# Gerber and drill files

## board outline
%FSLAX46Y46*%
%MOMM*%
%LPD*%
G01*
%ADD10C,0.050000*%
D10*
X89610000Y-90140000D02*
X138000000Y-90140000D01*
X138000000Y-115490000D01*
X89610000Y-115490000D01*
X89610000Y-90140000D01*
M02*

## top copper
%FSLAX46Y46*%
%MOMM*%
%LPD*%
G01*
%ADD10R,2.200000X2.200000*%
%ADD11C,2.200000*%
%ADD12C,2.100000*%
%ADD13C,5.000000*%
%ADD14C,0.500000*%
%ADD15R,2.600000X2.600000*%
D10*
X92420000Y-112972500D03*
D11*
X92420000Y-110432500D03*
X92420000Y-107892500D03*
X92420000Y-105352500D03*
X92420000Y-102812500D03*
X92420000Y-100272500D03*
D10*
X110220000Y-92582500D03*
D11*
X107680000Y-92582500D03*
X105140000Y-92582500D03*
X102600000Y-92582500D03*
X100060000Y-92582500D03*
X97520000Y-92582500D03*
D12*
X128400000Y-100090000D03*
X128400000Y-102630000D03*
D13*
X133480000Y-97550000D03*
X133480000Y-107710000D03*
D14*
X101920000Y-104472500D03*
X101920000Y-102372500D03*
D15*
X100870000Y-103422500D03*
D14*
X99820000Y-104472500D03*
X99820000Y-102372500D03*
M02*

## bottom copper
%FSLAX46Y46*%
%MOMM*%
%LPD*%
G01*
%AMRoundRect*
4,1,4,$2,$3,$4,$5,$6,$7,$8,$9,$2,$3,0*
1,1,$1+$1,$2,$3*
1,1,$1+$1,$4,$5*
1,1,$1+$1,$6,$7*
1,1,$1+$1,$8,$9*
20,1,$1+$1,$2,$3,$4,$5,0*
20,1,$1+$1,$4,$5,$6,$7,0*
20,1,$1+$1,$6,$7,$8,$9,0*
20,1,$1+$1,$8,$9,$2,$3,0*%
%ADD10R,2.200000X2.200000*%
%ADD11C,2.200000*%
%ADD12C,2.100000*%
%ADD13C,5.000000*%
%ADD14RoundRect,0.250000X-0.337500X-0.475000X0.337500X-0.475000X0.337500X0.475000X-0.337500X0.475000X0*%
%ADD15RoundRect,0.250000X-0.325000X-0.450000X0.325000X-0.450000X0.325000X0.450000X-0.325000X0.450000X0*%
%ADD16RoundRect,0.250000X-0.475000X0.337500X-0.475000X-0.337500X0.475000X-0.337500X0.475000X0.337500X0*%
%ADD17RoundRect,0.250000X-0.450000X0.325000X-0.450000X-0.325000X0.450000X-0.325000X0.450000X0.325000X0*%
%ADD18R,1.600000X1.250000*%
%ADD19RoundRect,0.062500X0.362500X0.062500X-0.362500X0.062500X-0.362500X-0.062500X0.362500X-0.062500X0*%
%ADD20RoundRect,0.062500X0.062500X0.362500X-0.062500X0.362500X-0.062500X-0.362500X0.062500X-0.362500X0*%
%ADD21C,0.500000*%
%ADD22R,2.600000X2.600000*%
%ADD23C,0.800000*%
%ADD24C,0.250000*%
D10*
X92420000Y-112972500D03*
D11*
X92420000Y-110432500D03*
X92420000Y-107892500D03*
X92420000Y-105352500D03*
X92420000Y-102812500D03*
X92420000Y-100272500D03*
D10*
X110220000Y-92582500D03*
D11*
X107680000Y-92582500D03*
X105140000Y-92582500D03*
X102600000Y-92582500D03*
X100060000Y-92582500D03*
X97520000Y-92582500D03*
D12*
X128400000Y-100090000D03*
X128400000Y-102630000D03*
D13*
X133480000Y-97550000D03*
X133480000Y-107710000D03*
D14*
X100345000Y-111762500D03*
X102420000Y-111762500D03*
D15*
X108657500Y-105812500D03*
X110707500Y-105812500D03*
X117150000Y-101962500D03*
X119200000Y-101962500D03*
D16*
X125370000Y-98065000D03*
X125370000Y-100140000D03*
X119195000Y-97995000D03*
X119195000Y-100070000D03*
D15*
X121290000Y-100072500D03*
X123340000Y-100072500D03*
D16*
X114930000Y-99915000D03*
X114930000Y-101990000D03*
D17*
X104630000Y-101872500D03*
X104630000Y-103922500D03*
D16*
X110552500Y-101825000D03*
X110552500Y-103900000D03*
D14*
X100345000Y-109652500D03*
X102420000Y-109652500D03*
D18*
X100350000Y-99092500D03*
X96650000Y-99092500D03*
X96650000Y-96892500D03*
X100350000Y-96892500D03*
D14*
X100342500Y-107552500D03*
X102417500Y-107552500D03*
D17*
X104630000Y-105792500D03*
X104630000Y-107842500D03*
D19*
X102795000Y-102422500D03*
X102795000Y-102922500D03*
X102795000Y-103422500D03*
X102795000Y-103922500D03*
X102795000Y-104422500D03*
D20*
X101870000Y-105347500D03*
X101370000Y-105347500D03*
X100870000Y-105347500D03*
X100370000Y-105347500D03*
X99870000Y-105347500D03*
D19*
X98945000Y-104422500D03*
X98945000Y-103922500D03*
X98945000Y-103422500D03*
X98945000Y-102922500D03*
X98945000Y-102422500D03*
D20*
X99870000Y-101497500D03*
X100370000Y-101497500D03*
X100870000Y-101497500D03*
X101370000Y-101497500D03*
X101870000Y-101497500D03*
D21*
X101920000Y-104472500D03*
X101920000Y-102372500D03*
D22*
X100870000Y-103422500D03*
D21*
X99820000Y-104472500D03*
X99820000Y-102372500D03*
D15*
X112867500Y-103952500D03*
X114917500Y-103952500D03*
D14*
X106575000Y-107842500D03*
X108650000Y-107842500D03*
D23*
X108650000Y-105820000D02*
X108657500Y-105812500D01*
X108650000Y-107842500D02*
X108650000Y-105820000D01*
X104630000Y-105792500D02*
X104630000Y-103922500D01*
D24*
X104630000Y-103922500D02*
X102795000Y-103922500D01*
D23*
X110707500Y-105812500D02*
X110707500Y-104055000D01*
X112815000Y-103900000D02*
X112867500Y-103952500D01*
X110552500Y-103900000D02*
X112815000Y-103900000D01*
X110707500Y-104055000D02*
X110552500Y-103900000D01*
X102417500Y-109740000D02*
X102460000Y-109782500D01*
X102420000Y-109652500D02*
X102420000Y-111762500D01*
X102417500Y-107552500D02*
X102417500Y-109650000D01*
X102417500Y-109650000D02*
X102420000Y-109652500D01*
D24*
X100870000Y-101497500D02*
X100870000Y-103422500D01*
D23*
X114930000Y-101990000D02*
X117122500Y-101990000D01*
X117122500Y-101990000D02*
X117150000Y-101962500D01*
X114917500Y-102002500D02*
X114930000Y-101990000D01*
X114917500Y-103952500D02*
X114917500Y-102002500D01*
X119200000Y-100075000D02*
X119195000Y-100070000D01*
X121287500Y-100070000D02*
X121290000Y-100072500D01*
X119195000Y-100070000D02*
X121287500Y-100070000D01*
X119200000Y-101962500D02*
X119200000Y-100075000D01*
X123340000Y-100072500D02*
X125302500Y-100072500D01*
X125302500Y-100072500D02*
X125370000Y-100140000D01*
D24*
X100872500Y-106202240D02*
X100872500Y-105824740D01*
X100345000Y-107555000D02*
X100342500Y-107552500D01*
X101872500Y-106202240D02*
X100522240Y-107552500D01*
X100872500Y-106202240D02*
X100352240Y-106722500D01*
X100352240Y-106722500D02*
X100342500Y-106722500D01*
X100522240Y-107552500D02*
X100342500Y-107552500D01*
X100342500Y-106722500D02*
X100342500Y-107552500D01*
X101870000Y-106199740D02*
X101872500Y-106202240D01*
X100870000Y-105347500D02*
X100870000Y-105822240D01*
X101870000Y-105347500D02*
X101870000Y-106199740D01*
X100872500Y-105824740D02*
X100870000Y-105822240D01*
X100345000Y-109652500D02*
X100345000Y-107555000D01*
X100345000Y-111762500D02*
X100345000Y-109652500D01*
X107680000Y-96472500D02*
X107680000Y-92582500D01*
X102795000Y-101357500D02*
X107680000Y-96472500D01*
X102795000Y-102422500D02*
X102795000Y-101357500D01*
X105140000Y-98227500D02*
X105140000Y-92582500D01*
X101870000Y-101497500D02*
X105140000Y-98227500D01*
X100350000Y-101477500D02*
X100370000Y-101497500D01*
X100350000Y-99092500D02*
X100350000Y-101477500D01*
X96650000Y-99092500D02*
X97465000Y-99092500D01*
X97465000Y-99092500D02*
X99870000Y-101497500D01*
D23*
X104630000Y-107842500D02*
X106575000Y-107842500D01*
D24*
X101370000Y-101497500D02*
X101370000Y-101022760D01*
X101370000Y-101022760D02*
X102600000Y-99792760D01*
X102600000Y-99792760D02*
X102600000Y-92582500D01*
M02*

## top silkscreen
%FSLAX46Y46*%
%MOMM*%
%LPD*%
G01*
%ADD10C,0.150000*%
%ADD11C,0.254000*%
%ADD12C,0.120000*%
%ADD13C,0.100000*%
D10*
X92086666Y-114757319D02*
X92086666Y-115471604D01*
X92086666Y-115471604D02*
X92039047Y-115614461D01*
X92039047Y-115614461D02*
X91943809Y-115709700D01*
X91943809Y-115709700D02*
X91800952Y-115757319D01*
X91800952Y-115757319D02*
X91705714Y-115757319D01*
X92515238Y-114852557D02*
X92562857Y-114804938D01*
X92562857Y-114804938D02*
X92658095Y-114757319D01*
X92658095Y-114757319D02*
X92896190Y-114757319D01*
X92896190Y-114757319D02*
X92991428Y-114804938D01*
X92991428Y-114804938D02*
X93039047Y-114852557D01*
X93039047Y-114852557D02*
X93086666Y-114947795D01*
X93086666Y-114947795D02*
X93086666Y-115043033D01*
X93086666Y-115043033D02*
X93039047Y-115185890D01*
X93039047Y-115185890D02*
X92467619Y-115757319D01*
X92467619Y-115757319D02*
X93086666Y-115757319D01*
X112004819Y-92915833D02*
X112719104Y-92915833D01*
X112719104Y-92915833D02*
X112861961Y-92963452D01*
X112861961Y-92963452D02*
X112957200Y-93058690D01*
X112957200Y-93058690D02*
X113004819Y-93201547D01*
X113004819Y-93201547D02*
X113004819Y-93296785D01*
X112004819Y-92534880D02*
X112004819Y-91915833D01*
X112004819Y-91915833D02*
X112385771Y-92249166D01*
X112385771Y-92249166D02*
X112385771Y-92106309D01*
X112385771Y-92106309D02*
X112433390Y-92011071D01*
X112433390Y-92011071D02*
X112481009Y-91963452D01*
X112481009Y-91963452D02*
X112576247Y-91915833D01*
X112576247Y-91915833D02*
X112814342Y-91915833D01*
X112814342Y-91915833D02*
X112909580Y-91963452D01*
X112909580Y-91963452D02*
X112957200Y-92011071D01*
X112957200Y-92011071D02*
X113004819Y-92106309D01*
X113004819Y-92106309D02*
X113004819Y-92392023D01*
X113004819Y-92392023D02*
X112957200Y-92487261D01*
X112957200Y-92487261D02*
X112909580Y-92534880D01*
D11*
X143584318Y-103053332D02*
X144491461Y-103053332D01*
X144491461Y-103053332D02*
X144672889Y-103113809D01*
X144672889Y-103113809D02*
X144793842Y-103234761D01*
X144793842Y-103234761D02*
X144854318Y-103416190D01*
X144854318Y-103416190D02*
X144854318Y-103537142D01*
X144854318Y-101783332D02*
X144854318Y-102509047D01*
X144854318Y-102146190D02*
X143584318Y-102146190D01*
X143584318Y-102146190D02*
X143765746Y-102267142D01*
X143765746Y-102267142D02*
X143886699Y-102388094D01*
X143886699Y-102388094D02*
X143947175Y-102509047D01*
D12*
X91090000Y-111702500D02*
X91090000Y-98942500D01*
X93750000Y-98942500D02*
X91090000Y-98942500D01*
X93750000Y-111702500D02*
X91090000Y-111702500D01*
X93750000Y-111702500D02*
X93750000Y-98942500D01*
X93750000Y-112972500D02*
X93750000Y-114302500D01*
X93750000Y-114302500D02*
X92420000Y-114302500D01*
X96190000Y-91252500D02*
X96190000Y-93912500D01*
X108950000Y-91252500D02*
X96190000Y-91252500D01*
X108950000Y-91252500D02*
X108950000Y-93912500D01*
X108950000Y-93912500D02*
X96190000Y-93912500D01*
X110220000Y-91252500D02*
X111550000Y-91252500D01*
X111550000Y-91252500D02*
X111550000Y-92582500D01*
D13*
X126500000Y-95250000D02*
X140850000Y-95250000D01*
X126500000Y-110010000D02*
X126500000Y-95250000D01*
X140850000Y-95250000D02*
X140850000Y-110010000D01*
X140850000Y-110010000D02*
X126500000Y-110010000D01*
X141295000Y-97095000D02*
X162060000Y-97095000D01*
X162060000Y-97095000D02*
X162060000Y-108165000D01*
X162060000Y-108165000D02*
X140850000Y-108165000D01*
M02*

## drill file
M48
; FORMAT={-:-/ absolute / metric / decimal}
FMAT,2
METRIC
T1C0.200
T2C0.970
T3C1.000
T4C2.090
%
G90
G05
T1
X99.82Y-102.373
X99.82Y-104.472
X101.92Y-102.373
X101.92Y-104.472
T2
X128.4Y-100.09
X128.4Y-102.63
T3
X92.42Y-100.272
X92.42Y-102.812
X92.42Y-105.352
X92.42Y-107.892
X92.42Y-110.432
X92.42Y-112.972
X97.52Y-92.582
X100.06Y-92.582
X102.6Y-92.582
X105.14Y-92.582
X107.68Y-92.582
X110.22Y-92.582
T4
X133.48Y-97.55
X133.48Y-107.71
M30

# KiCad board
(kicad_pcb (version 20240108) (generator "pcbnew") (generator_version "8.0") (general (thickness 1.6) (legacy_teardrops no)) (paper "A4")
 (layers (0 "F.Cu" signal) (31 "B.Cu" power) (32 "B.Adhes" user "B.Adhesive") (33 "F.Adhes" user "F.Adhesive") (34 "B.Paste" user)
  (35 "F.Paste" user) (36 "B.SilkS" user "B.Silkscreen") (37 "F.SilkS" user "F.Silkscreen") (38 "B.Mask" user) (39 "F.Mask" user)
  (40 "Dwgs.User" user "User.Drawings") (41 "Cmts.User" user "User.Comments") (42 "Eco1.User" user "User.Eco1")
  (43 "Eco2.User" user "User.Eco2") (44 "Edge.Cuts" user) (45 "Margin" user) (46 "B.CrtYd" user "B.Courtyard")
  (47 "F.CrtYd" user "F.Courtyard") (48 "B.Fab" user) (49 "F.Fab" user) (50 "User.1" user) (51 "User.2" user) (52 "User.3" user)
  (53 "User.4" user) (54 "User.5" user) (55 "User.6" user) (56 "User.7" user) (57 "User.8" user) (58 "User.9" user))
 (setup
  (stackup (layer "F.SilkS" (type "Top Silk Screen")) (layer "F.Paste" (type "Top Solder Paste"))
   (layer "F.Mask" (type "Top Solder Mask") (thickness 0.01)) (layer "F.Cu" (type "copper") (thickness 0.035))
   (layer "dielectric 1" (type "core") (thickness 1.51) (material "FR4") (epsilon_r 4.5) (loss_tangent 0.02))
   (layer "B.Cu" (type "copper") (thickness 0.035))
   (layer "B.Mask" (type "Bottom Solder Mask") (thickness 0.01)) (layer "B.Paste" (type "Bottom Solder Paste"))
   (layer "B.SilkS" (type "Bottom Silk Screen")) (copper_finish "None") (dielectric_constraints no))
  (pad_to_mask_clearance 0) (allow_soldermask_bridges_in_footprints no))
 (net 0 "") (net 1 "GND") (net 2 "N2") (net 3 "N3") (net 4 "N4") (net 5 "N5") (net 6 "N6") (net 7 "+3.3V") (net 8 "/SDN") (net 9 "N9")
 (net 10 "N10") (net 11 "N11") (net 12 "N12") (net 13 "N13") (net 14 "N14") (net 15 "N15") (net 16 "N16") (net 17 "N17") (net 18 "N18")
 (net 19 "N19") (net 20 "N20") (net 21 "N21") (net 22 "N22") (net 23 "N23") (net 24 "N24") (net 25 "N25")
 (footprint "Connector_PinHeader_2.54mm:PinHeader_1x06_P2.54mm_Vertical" (layer "F.Cu") (at 92.42 112.9725 180)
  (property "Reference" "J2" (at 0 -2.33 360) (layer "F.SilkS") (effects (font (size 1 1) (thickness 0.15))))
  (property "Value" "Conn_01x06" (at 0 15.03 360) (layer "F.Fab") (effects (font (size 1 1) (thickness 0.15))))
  (fp_line (start 1.33 1.27) (end 1.33 14.03) (stroke (width 0.12) (type solid)) (layer "F.SilkS"))
  (fp_line (start -1.33 14.03) (end 1.33 14.03) (stroke (width 0.12) (type solid)) (layer "F.SilkS"))
  (fp_line (start -1.33 1.27) (end 1.33 1.27) (stroke (width 0.12) (type solid)) (layer "F.SilkS"))
  (fp_line (start -1.33 1.27) (end -1.33 14.03) (stroke (width 0.12) (type solid)) (layer "F.SilkS"))
  (fp_line (start -1.33 0) (end -1.33 -1.33) (stroke (width 0.12) (type solid)) (layer "F.SilkS"))
  (fp_line (start -1.33 -1.33) (end 0 -1.33) (stroke (width 0.12) (type solid)) (layer "F.SilkS"))
  (pad "1" thru_hole rect (at 0 0 180) (size 2.2 2.2) (drill 1) (layers "*.Cu" "*.Mask") (remove_unused_layers no) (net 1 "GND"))
  (pad "2" thru_hole circle (at 0 2.54 180) (size 2.2 2.2) (drill 1) (layers "*.Cu" "*.Mask") (remove_unused_layers no) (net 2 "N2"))
  (pad "3" thru_hole circle (at 0 5.08 180) (size 2.2 2.2) (drill 1) (layers "*.Cu" "*.Mask") (remove_unused_layers no) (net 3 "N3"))
  (pad "4" thru_hole circle (at 0 7.62 180) (size 2.2 2.2) (drill 1) (layers "*.Cu" "*.Mask") (remove_unused_layers no) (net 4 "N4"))
  (pad "5" thru_hole circle (at 0 10.16 180) (size 2.2 2.2) (drill 1) (layers "*.Cu" "*.Mask") (remove_unused_layers no) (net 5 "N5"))
  (pad "6" thru_hole circle (at 0 12.7 180) (size 2.2 2.2) (drill 1) (layers "*.Cu" "*.Mask") (remove_unused_layers no) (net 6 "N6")))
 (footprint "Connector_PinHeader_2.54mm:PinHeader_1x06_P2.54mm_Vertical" (layer "F.Cu") (at 110.22 92.5825 -90)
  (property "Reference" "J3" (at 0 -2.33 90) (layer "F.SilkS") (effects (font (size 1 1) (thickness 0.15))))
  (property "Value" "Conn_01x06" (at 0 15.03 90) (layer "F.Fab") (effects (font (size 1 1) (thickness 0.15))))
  (fp_line (start -1.33 14.03) (end 1.33 14.03) (stroke (width 0.12) (type solid)) (layer "F.SilkS"))
  (fp_line (start -1.33 1.27) (end -1.33 14.03) (stroke (width 0.12) (type solid)) (layer "F.SilkS"))
  (fp_line (start -1.33 1.27) (end 1.33 1.27) (stroke (width 0.12) (type solid)) (layer "F.SilkS"))
  (fp_line (start 1.33 1.27) (end 1.33 14.03) (stroke (width 0.12) (type solid)) (layer "F.SilkS"))
  (fp_line (start -1.33 0) (end -1.33 -1.33) (stroke (width 0.12) (type solid)) (layer "F.SilkS"))
  (fp_line (start -1.33 -1.33) (end 0 -1.33) (stroke (width 0.12) (type solid)) (layer "F.SilkS"))
  (pad "1" thru_hole rect (at 0 0 270) (size 2.2 2.2) (drill 1) (layers "*.Cu" "*.Mask") (remove_unused_layers no) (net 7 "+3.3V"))
  (pad "2" thru_hole circle (at 0 2.54 270) (size 2.2 2.2) (drill 1) (layers "*.Cu" "*.Mask") (remove_unused_layers no) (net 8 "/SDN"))
  (pad "3" thru_hole circle (at 0 5.08 270) (size 2.2 2.2) (drill 1) (layers "*.Cu" "*.Mask") (remove_unused_layers no) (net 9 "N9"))
  (pad "4" thru_hole circle (at 0 7.62 270) (size 2.2 2.2) (drill 1) (layers "*.Cu" "*.Mask") (remove_unused_layers no) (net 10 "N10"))
  (pad "5" thru_hole circle (at 0 10.16 270) (size 2.2 2.2) (drill 1) (layers "*.Cu" "*.Mask") (remove_unused_layers no) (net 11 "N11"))
  (pad "6" thru_hole circle (at 0 12.7 270) (size 2.2 2.2) (drill 1) (layers "*.Cu" "*.Mask") (remove_unused_layers no) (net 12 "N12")))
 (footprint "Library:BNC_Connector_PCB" (layer "F.Cu") (at 128.4 100.09 -90)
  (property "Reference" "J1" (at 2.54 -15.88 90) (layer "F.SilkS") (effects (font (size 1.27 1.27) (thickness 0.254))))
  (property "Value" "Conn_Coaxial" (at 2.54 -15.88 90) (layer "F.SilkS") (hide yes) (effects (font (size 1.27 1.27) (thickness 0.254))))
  (fp_line (start -4.84 1.9) (end -4.84 -12.45) (stroke (width 0.1) (type solid)) (layer "F.SilkS"))
  (fp_line (start 9.92 1.9) (end -4.84 1.9) (stroke (width 0.1) (type solid)) (layer "F.SilkS"))
  (fp_line (start -4.84 -12.45) (end 9.92 -12.45) (stroke (width 0.1) (type solid)) (layer "F.SilkS"))
  (fp_line (start 9.92 -12.45) (end 9.92 1.9) (stroke (width 0.1) (type solid)) (layer "F.SilkS"))
  (fp_line (start -2.995 -12.895) (end -2.995 -33.66) (stroke (width 0.1) (type solid)) (layer "F.SilkS"))
  (fp_line (start -2.995 -33.66) (end 8.075 -33.66) (stroke (width 0.1) (type solid)) (layer "F.SilkS"))
  (fp_line (start 8.075 -33.66) (end 8.075 -12.45) (stroke (width 0.1) (type solid)) (layer "F.SilkS"))
  (pad "1" thru_hole circle (at 0 0 270) (size 2.1 2.1) (drill 0.97) (layers "*.Cu" "*.Mask") (remove_unused_layers no) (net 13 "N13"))
  (pad "2" thru_hole circle (at 2.54 0 270) (size 2.1 2.1) (drill 0.97) (layers "*.Cu" "*.Mask") (remove_unused_layers no) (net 1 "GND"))
  (pad "MH1" thru_hole circle (at -2.54 -5.08 270) (size 5 5) (drill 2.09) (layers "*.Cu" "*.Mask") (remove_unused_layers no))
  (pad "MH2" thru_hole circle (at 7.62 -5.08 270) (size 5 5) (drill 2.09) (layers "*.Cu" "*.Mask") (remove_unused_layers no)))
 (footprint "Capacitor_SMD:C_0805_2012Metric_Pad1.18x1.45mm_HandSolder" (layer "B.Cu") (at 101.3825 111.7625)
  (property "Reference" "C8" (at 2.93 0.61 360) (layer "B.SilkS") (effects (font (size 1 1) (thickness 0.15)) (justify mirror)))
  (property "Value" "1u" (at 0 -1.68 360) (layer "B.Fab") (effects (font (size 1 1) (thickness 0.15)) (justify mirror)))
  (pad "1" smd roundrect (at -1.0375 0) (size 1.175 1.45) (layers "B.Cu" "B.Paste" "B.Mask") (roundrect_rratio 0.212766) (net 7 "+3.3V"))
  (pad "2" smd roundrect (at 1.0375 0) (size 1.175 1.45) (layers "B.Cu" "B.Paste" "B.Mask") (roundrect_rratio 0.212766) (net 1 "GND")))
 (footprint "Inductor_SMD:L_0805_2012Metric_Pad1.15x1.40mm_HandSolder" (layer "B.Cu") (at 109.6825 105.8125)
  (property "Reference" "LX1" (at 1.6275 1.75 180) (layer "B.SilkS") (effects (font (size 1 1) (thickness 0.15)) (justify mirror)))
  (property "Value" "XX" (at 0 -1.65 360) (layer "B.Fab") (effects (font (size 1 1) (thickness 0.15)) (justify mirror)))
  (pad "1" smd roundrect (at -1.025 0) (size 1.15 1.4) (layers "B.Cu" "B.Paste" "B.Mask") (roundrect_rratio 0.217391) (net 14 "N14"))
  (pad "2" smd roundrect (at 1.025 0) (size 1.15 1.4) (layers "B.Cu" "B.Paste" "B.Mask") (roundrect_rratio 0.217391) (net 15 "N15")))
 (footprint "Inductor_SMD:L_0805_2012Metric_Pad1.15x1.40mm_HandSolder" (layer "B.Cu") (at 118.175 101.9625)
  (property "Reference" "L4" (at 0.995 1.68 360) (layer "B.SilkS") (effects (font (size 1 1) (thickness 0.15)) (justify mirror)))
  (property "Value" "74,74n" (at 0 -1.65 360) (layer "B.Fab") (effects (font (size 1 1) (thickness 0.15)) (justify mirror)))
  (pad "1" smd roundrect (at -1.025 0) (size 1.15 1.4) (layers "B.Cu" "B.Paste" "B.Mask") (roundrect_rratio 0.217391) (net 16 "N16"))
  (pad "2" smd roundrect (at 1.025 0) (size 1.15 1.4) (layers "B.Cu" "B.Paste" "B.Mask") (roundrect_rratio 0.217391) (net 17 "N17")))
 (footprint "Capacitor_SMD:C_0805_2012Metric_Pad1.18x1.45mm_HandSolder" (layer "B.Cu") (at 125.37 99.1025 -90)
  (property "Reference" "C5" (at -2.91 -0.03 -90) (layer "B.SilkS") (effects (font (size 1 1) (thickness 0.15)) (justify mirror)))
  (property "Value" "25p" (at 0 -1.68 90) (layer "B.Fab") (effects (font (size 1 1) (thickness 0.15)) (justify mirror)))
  (pad "1" smd roundrect (at -1.0375 0 270) (size 1.175 1.45) (layers "B.Cu" "B.Paste" "B.Mask") (roundrect_rratio 0.212766) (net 1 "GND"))
  (pad "2" smd roundrect (at 1.0375 0 270) (size 1.175 1.45) (layers "B.Cu" "B.Paste" "B.Mask") (roundrect_rratio 0.212766) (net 13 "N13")))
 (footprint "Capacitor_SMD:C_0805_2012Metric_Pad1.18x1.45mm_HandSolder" (layer "B.Cu") (at 119.195 99.0325 -90)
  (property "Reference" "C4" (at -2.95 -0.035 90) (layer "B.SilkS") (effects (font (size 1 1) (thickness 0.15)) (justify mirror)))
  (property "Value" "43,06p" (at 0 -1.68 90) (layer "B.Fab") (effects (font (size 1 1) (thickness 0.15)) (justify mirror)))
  (pad "1" smd roundrect (at -1.0375 0 270) (size 1.175 1.45) (layers "B.Cu" "B.Paste" "B.Mask") (roundrect_rratio 0.212766) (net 1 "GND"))
  (pad "2" smd roundrect (at 1.0375 0 270) (size 1.175 1.45) (layers "B.Cu" "B.Paste" "B.Mask") (roundrect_rratio 0.212766) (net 17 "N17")))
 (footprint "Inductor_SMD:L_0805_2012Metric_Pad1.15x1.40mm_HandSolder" (layer "B.Cu") (at 122.315 100.0725)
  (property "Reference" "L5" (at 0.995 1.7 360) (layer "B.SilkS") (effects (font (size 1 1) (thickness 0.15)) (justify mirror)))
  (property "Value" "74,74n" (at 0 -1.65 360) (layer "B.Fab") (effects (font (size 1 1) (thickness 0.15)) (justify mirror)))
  (pad "1" smd roundrect (at -1.025 0) (size 1.15 1.4) (layers "B.Cu" "B.Paste" "B.Mask") (roundrect_rratio 0.217391) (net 17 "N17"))
  (pad "2" smd roundrect (at 1.025 0) (size 1.15 1.4) (layers "B.Cu" "B.Paste" "B.Mask") (roundrect_rratio 0.217391) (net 13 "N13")))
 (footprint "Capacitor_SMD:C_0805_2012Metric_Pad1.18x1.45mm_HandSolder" (layer "B.Cu") (at 114.93 100.9525 -90)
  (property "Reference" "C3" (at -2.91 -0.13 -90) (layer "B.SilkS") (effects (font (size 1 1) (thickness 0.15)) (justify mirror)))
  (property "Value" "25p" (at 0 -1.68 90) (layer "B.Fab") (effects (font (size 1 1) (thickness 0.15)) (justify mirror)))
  (pad "1" smd roundrect (at -1.0375 0 270) (size 1.175 1.45) (layers "B.Cu" "B.Paste" "B.Mask") (roundrect_rratio 0.212766) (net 1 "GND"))
  (pad "2" smd roundrect (at 1.0375 0 270) (size 1.175 1.45) (layers "B.Cu" "B.Paste" "B.Mask") (roundrect_rratio 0.212766) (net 16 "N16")))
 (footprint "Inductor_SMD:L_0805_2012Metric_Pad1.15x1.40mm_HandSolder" (layer "B.Cu") (at 104.63 102.8975 -90)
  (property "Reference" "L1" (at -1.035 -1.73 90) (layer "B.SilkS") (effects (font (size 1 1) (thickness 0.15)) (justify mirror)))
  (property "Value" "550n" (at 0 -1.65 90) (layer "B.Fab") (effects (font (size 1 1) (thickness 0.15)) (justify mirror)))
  (pad "1" smd roundrect (at -1.025 0 270) (size 1.15 1.4) (layers "B.Cu" "B.Paste" "B.Mask") (roundrect_rratio 0.217391) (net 7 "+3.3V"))
  (pad "2" smd roundrect (at 1.025 0 270) (size 1.15 1.4) (layers "B.Cu" "B.Paste" "B.Mask") (roundrect_rratio 0.217391) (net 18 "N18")))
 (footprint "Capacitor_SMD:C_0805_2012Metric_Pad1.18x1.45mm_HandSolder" (layer "B.Cu") (at 110.5525 102.8625 -90)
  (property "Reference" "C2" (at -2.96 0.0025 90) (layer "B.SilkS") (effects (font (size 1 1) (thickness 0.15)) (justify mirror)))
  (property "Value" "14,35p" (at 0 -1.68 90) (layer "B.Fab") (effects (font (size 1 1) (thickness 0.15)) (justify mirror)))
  (pad "1" smd roundrect (at -1.0375 0 270) (size 1.175 1.45) (layers "B.Cu" "B.Paste" "B.Mask") (roundrect_rratio 0.212766) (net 1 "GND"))
  (pad "2" smd roundrect (at 1.0375 0 270) (size 1.175 1.45) (layers "B.Cu" "B.Paste" "B.Mask") (roundrect_rratio 0.212766) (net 15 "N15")))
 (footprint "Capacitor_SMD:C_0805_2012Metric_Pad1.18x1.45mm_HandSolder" (layer "B.Cu") (at 101.3825 109.6525)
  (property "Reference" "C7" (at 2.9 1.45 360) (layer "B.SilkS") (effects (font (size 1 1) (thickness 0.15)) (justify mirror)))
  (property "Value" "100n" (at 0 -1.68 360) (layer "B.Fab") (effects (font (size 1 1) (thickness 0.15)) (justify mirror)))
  (pad "1" smd roundrect (at -1.0375 0) (size 1.175 1.45) (layers "B.Cu" "B.Paste" "B.Mask") (roundrect_rratio 0.212766) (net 7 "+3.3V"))
  (pad "2" smd roundrect (at 1.0375 0) (size 1.175 1.45) (layers "B.Cu" "B.Paste" "B.Mask") (roundrect_rratio 0.212766) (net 1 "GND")))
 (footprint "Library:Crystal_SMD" (layer "B.Cu") (at 98.5 97.9925 180)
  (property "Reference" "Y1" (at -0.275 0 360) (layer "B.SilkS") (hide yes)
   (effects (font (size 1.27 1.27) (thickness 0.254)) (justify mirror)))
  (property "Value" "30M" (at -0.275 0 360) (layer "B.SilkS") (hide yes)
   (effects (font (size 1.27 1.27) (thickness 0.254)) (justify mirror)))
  (pad "1" smd rect (at -1.85 -1.1 90) (size 1.25 1.6) (layers "B.Cu" "B.Paste" "B.Mask") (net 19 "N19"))
  (pad "2" smd rect (at 1.85 -1.1 90) (size 1.25 1.6) (layers "B.Cu" "B.Paste" "B.Mask") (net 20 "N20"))
  (pad "3" smd rect (at 1.85 1.1 90) (size 1.25 1.6) (layers "B.Cu" "B.Paste" "B.Mask"))
  (pad "4" smd rect (at -1.85 1.1 90) (size 1.25 1.6) (layers "B.Cu" "B.Paste" "B.Mask")))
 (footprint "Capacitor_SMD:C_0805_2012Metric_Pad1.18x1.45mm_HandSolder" (layer "B.Cu") (at 101.38 107.5525)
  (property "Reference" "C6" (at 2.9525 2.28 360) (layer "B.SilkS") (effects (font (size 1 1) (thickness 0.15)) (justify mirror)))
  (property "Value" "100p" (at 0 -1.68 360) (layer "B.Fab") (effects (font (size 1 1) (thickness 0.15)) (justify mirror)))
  (pad "1" smd roundrect (at -1.0375 0) (size 1.175 1.45) (layers "B.Cu" "B.Paste" "B.Mask") (roundrect_rratio 0.212766) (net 7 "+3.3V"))
  (pad "2" smd roundrect (at 1.0375 0) (size 1.175 1.45) (layers "B.Cu" "B.Paste" "B.Mask") (roundrect_rratio 0.212766) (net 1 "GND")))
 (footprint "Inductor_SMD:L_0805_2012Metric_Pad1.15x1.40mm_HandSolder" (layer "B.Cu") (at 104.63 106.8175 -90)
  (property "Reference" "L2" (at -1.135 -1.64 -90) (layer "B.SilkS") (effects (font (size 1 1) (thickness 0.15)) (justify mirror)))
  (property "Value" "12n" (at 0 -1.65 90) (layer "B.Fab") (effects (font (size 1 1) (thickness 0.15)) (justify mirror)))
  (pad "1" smd roundrect (at -1.025 0 270) (size 1.15 1.4) (layers "B.Cu" "B.Paste" "B.Mask") (roundrect_rratio 0.217391) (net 18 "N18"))
  (pad "2" smd roundrect (at 1.025 0 270) (size 1.15 1.4) (layers "B.Cu" "B.Paste" "B.Mask") (roundrect_rratio 0.217391) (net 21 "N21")))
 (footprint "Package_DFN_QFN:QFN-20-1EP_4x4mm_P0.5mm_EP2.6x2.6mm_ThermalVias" (layer "B.Cu") (at 100.87 103.4225 180)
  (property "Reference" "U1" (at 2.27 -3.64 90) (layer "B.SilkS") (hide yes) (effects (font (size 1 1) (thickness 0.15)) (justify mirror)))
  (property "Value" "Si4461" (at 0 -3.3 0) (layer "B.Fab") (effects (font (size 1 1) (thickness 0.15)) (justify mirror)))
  (pad "" smd roundrect (at -0.65 -0.65 180) (size 1.13 1.13) (layers "B.Paste") (roundrect_rratio 0.221239))
  (pad "" smd roundrect (at -0.65 0.65 180) (size 1.13 1.13) (layers "B.Paste") (roundrect_rratio 0.221239))
  (pad "" smd roundrect (at 0.65 -0.65 180) (size 1.13 1.13) (layers "B.Paste") (roundrect_rratio 0.221239))
  (pad "" smd roundrect (at 0.65 0.65 180) (size 1.13 1.13) (layers "B.Paste") (roundrect_rratio 0.221239))
  (pad "1" smd roundrect (at -1.925 1 180) (size 0.85 0.25) (layers "B.Cu" "B.Paste" "B.Mask") (roundrect_rratio 0.25) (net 8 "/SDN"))
  (pad "2" smd roundrect (at -1.925 0.5 180) (size 0.85 0.25) (layers "B.Cu" "B.Paste" "B.Mask") (roundrect_rratio 0.25) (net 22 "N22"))
  (pad "3" smd roundrect (at -1.925 0 180) (size 0.85 0.25) (layers "B.Cu" "B.Paste" "B.Mask") (roundrect_rratio 0.25) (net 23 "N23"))
  (pad "4" smd roundrect (at -1.925 -0.5 180) (size 0.85 0.25) (layers "B.Cu" "B.Paste" "B.Mask") (roundrect_rratio 0.25) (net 18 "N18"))
  (pad "5" smd roundrect (at -1.925 -1 180) (size 0.85 0.25) (layers "B.Cu" "B.Paste" "B.Mask") (roundrect_rratio 0.25) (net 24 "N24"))
  (pad "6" smd roundrect (at -1 -1.925 180) (size 0.25 0.85) (layers "B.Cu" "B.Paste" "B.Mask") (roundrect_rratio 0.25) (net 7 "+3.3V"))
  (pad "7" smd roundrect (at -0.5 -1.925 180) (size 0.25 0.85) (layers "B.Cu" "B.Paste" "B.Mask") (roundrect_rratio 0.25) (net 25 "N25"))
  (pad "8" smd roundrect (at 0 -1.925 180) (size 0.25 0.85) (layers "B.Cu" "B.Paste" "B.Mask") (roundrect_rratio 0.25) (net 7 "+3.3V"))
  (pad "9" smd roundrect (at 0.5 -1.925 180) (size 0.25 0.85) (layers "B.Cu" "B.Paste" "B.Mask") (roundrect_rratio 0.25) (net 12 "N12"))
  (pad "10" smd roundrect (at 1 -1.925 180) (size 0.25 0.85) (layers "B.Cu" "B.Paste" "B.Mask") (roundrect_rratio 0.25) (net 11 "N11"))
  (pad "11" smd roundrect (at 1.925 -1 180) (size 0.85 0.25) (layers "B.Cu" "B.Paste" "B.Mask") (roundrect_rratio 0.25) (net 2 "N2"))
  (pad "12" smd roundrect (at 1.925 -0.5 180) (size 0.85 0.25) (layers "B.Cu" "B.Paste" "B.Mask") (roundrect_rratio 0.25) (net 3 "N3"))
  (pad "13" smd roundrect (at 1.925 0 180) (size 0.85 0.25) (layers "B.Cu" "B.Paste" "B.Mask") (roundrect_rratio 0.25) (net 4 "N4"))
  (pad "14" smd roundrect (at 1.925 0.5 180) (size 0.85 0.25) (layers "B.Cu" "B.Paste" "B.Mask") (roundrect_rratio 0.25) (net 5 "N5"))
  (pad "15" smd roundrect (at 1.925 1 180) (size 0.85 0.25) (layers "B.Cu" "B.Paste" "B.Mask") (roundrect_rratio 0.25) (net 6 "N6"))
  (pad "16" smd roundrect (at 1 1.925 180) (size 0.25 0.85) (layers "B.Cu" "B.Paste" "B.Mask") (roundrect_rratio 0.25) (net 20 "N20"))
  (pad "17" smd roundrect (at 0.5 1.925 180) (size 0.25 0.85) (layers "B.Cu" "B.Paste" "B.Mask") (roundrect_rratio 0.25) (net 19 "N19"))
  (pad "18" smd roundrect (at 0 1.925 180) (size 0.25 0.85) (layers "B.Cu" "B.Paste" "B.Mask") (roundrect_rratio 0.25) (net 1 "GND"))
  (pad "19" smd roundrect (at -0.5 1.925 180) (size 0.25 0.85) (layers "B.Cu" "B.Paste" "B.Mask") (roundrect_rratio 0.25) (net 10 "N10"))
  (pad "20" smd roundrect (at -1 1.925 180) (size 0.25 0.85) (layers "B.Cu" "B.Paste" "B.Mask") (roundrect_rratio 0.25) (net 9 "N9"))
  (pad "21" thru_hole circle (at -1.05 -1.05 180) (size 0.5 0.5) (drill 0.2) (layers "*.Cu") (remove_unused_layers no) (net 1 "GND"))
  (pad "21" thru_hole circle (at -1.05 1.05 180) (size 0.5 0.5) (drill 0.2) (layers "*.Cu") (remove_unused_layers no) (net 1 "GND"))
  (pad "21" smd rect (at 0 0 180) (size 2.6 2.6) (layers "F.Cu") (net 1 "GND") (zone_connect 2))
  (pad "21" smd rect (at 0 0 180) (size 2.6 2.6) (layers "B.Cu" "B.Mask") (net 1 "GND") (zone_connect 2))
  (pad "21" thru_hole circle (at 1.05 -1.05 180) (size 0.5 0.5) (drill 0.2) (layers "*.Cu") (remove_unused_layers no) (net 1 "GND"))
  (pad "21" thru_hole circle (at 1.05 1.05 180) (size 0.5 0.5) (drill 0.2) (layers "*.Cu") (remove_unused_layers no) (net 1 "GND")))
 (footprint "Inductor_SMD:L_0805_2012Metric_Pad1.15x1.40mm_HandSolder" (layer "B.Cu") (at 113.8925 103.9525)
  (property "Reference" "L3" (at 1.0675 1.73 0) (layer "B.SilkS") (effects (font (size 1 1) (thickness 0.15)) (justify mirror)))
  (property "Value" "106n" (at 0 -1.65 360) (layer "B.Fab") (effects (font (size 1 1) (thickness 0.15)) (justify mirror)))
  (pad "1" smd roundrect (at -1.025 0) (size 1.15 1.4) (layers "B.Cu" "B.Paste" "B.Mask") (roundrect_rratio 0.217391) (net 15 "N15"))
  (pad "2" smd roundrect (at 1.025 0) (size 1.15 1.4) (layers "B.Cu" "B.Paste" "B.Mask") (roundrect_rratio 0.217391) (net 16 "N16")))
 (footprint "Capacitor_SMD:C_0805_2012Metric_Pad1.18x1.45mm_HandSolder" (layer "B.Cu") (at 107.6125 107.8425)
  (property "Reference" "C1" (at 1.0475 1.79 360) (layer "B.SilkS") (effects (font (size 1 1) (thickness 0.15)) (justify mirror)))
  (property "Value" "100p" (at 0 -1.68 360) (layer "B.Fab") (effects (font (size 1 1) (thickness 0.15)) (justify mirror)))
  (pad "1" smd roundrect (at -1.0375 0) (size 1.175 1.45) (layers "B.Cu" "B.Paste" "B.Mask") (roundrect_rratio 0.212766) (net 21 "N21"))
  (pad "2" smd roundrect (at 1.0375 0) (size 1.175 1.45) (layers "B.Cu" "B.Paste" "B.Mask") (roundrect_rratio 0.212766) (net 14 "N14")))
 (gr_rect (start 89.61 90.14) (end 138 115.49) (stroke (width 0.05) (type default)) (fill none) (layer "Edge.Cuts"))
 (segment (start 108.65 105.82) (end 108.6575 105.8125) (width 0.8) (layer "B.Cu") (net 14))
 (segment (start 108.65 107.8425) (end 108.65 105.82) (width 0.8) (layer "B.Cu") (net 14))
 (segment (start 104.63 105.7925) (end 104.63 103.9225) (width 0.8) (layer "B.Cu") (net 18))
 (segment (start 104.63 103.9225) (end 102.795 103.9225) (width 0.25) (layer "B.Cu") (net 18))
 (segment (start 110.7075 105.8125) (end 110.7075 104.055) (width 0.8) (layer "B.Cu") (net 15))
 (segment (start 112.815 103.9) (end 112.8675 103.9525) (width 0.8) (layer "B.Cu") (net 15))
 (segment (start 110.5525 103.9) (end 112.815 103.9) (width 0.8) (layer "B.Cu") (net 15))
 (segment (start 110.7075 104.055) (end 110.5525 103.9) (width 0.8) (layer "B.Cu") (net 15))
 (segment (start 102.4175 109.74) (end 102.46 109.7825) (width 0.8) (layer "B.Cu") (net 1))
 (segment (start 102.42 109.6525) (end 102.42 111.7625) (width 0.8) (layer "B.Cu") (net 1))
 (segment (start 102.4175 107.5525) (end 102.4175 109.65) (width 0.8) (layer "B.Cu") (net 1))
 (segment (start 102.4175 109.65) (end 102.42 109.6525) (width 0.8) (layer "B.Cu") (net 1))
 (segment (start 100.87 101.4975) (end 100.87 103.4225) (width 0.25) (layer "B.Cu") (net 1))
 (segment (start 114.93 101.99) (end 117.1225 101.99) (width 0.8) (layer "B.Cu") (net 16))
 (segment (start 117.1225 101.99) (end 117.15 101.9625) (width 0.8) (layer "B.Cu") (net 16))
 (segment (start 114.9175 102.0025) (end 114.93 101.99) (width 0.8) (layer "B.Cu") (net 16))
 (segment (start 114.9175 103.9525) (end 114.9175 102.0025) (width 0.8) (layer "B.Cu") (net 16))
 (segment (start 119.2 100.075) (end 119.195 100.07) (width 0.8) (layer "B.Cu") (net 17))
 (segment (start 121.2875 100.07) (end 121.29 100.0725) (width 0.8) (layer "B.Cu") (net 17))
 (segment (start 119.195 100.07) (end 121.2875 100.07) (width 0.8) (layer "B.Cu") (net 17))
 (segment (start 119.2 101.9625) (end 119.2 100.075) (width 0.8) (layer "B.Cu") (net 17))
 (segment (start 123.34 100.0725) (end 125.3025 100.0725) (width 0.8) (layer "B.Cu") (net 13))
 (segment (start 125.3025 100.0725) (end 125.37 100.14) (width 0.8) (layer "B.Cu") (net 13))
 (segment (start 100.8725 106.20224) (end 100.8725 105.82474) (width 0.25) (layer "B.Cu") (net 7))
 (segment (start 100.345 107.555) (end 100.3425 107.5525) (width 0.25) (layer "B.Cu") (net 7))
 (segment (start 101.8725 106.20224) (end 100.52224 107.5525) (width 0.25) (layer "B.Cu") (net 7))
 (segment (start 100.8725 106.20224) (end 100.35224 106.7225) (width 0.25) (layer "B.Cu") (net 7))
 (segment (start 100.35224 106.7225) (end 100.3425 106.7225) (width 0.25) (layer "B.Cu") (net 7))
 (segment (start 100.52224 107.5525) (end 100.3425 107.5525) (width 0.25) (layer "B.Cu") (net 7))
 (segment (start 100.3425 106.7225) (end 100.3425 107.5525) (width 0.25) (layer "B.Cu") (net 7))
 (segment (start 101.87 106.19974) (end 101.8725 106.20224) (width 0.25) (layer "B.Cu") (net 7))
 (segment (start 100.87 105.3475) (end 100.87 105.82224) (width 0.25) (layer "B.Cu") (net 7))
 (segment (start 101.87 105.3475) (end 101.87 106.19974) (width 0.25) (layer "B.Cu") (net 7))
 (segment (start 100.8725 105.82474) (end 100.87 105.82224) (width 0.25) (layer "B.Cu") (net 7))
 (segment (start 100.345 109.6525) (end 100.345 107.555) (width 0.25) (layer "B.Cu") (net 7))
 (segment (start 100.345 111.7625) (end 100.345 109.6525) (width 0.25) (layer "B.Cu") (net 7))
 (segment (start 107.68 96.4725) (end 107.68 92.5825) (width 0.25) (layer "B.Cu") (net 8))
 (segment (start 102.795 101.3575) (end 107.68 96.4725) (width 0.25) (layer "B.Cu") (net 8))
 (segment (start 102.795 102.4225) (end 102.795 101.3575) (width 0.25) (layer "B.Cu") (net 8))
 (segment (start 105.14 98.2275) (end 105.14 92.5825) (width 0.25) (layer "B.Cu") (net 9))
 (segment (start 101.87 101.4975) (end 105.14 98.2275) (width 0.25) (layer "B.Cu") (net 9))
 (segment (start 100.35 101.4775) (end 100.37 101.4975) (width 0.25) (layer "B.Cu") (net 19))
 (segment (start 100.35 99.0925) (end 100.35 101.4775) (width 0.25) (layer "B.Cu") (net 19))
 (segment (start 96.65 99.0925) (end 97.465 99.0925) (width 0.25) (layer "B.Cu") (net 20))
 (segment (start 97.465 99.0925) (end 99.87 101.4975) (width 0.25) (layer "B.Cu") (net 20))
 (segment (start 104.63 107.8425) (end 106.575 107.8425) (width 0.8) (layer "B.Cu") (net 21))
 (segment (start 101.37 101.4975) (end 101.37 101.02276) (width 0.25) (layer "B.Cu") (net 10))
 (segment (start 101.37 101.02276) (end 102.6 99.79276) (width 0.25) (layer "B.Cu") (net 10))
 (segment (start 102.6 99.79276) (end 102.6 92.5825) (width 0.25) (layer "B.Cu") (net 10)))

